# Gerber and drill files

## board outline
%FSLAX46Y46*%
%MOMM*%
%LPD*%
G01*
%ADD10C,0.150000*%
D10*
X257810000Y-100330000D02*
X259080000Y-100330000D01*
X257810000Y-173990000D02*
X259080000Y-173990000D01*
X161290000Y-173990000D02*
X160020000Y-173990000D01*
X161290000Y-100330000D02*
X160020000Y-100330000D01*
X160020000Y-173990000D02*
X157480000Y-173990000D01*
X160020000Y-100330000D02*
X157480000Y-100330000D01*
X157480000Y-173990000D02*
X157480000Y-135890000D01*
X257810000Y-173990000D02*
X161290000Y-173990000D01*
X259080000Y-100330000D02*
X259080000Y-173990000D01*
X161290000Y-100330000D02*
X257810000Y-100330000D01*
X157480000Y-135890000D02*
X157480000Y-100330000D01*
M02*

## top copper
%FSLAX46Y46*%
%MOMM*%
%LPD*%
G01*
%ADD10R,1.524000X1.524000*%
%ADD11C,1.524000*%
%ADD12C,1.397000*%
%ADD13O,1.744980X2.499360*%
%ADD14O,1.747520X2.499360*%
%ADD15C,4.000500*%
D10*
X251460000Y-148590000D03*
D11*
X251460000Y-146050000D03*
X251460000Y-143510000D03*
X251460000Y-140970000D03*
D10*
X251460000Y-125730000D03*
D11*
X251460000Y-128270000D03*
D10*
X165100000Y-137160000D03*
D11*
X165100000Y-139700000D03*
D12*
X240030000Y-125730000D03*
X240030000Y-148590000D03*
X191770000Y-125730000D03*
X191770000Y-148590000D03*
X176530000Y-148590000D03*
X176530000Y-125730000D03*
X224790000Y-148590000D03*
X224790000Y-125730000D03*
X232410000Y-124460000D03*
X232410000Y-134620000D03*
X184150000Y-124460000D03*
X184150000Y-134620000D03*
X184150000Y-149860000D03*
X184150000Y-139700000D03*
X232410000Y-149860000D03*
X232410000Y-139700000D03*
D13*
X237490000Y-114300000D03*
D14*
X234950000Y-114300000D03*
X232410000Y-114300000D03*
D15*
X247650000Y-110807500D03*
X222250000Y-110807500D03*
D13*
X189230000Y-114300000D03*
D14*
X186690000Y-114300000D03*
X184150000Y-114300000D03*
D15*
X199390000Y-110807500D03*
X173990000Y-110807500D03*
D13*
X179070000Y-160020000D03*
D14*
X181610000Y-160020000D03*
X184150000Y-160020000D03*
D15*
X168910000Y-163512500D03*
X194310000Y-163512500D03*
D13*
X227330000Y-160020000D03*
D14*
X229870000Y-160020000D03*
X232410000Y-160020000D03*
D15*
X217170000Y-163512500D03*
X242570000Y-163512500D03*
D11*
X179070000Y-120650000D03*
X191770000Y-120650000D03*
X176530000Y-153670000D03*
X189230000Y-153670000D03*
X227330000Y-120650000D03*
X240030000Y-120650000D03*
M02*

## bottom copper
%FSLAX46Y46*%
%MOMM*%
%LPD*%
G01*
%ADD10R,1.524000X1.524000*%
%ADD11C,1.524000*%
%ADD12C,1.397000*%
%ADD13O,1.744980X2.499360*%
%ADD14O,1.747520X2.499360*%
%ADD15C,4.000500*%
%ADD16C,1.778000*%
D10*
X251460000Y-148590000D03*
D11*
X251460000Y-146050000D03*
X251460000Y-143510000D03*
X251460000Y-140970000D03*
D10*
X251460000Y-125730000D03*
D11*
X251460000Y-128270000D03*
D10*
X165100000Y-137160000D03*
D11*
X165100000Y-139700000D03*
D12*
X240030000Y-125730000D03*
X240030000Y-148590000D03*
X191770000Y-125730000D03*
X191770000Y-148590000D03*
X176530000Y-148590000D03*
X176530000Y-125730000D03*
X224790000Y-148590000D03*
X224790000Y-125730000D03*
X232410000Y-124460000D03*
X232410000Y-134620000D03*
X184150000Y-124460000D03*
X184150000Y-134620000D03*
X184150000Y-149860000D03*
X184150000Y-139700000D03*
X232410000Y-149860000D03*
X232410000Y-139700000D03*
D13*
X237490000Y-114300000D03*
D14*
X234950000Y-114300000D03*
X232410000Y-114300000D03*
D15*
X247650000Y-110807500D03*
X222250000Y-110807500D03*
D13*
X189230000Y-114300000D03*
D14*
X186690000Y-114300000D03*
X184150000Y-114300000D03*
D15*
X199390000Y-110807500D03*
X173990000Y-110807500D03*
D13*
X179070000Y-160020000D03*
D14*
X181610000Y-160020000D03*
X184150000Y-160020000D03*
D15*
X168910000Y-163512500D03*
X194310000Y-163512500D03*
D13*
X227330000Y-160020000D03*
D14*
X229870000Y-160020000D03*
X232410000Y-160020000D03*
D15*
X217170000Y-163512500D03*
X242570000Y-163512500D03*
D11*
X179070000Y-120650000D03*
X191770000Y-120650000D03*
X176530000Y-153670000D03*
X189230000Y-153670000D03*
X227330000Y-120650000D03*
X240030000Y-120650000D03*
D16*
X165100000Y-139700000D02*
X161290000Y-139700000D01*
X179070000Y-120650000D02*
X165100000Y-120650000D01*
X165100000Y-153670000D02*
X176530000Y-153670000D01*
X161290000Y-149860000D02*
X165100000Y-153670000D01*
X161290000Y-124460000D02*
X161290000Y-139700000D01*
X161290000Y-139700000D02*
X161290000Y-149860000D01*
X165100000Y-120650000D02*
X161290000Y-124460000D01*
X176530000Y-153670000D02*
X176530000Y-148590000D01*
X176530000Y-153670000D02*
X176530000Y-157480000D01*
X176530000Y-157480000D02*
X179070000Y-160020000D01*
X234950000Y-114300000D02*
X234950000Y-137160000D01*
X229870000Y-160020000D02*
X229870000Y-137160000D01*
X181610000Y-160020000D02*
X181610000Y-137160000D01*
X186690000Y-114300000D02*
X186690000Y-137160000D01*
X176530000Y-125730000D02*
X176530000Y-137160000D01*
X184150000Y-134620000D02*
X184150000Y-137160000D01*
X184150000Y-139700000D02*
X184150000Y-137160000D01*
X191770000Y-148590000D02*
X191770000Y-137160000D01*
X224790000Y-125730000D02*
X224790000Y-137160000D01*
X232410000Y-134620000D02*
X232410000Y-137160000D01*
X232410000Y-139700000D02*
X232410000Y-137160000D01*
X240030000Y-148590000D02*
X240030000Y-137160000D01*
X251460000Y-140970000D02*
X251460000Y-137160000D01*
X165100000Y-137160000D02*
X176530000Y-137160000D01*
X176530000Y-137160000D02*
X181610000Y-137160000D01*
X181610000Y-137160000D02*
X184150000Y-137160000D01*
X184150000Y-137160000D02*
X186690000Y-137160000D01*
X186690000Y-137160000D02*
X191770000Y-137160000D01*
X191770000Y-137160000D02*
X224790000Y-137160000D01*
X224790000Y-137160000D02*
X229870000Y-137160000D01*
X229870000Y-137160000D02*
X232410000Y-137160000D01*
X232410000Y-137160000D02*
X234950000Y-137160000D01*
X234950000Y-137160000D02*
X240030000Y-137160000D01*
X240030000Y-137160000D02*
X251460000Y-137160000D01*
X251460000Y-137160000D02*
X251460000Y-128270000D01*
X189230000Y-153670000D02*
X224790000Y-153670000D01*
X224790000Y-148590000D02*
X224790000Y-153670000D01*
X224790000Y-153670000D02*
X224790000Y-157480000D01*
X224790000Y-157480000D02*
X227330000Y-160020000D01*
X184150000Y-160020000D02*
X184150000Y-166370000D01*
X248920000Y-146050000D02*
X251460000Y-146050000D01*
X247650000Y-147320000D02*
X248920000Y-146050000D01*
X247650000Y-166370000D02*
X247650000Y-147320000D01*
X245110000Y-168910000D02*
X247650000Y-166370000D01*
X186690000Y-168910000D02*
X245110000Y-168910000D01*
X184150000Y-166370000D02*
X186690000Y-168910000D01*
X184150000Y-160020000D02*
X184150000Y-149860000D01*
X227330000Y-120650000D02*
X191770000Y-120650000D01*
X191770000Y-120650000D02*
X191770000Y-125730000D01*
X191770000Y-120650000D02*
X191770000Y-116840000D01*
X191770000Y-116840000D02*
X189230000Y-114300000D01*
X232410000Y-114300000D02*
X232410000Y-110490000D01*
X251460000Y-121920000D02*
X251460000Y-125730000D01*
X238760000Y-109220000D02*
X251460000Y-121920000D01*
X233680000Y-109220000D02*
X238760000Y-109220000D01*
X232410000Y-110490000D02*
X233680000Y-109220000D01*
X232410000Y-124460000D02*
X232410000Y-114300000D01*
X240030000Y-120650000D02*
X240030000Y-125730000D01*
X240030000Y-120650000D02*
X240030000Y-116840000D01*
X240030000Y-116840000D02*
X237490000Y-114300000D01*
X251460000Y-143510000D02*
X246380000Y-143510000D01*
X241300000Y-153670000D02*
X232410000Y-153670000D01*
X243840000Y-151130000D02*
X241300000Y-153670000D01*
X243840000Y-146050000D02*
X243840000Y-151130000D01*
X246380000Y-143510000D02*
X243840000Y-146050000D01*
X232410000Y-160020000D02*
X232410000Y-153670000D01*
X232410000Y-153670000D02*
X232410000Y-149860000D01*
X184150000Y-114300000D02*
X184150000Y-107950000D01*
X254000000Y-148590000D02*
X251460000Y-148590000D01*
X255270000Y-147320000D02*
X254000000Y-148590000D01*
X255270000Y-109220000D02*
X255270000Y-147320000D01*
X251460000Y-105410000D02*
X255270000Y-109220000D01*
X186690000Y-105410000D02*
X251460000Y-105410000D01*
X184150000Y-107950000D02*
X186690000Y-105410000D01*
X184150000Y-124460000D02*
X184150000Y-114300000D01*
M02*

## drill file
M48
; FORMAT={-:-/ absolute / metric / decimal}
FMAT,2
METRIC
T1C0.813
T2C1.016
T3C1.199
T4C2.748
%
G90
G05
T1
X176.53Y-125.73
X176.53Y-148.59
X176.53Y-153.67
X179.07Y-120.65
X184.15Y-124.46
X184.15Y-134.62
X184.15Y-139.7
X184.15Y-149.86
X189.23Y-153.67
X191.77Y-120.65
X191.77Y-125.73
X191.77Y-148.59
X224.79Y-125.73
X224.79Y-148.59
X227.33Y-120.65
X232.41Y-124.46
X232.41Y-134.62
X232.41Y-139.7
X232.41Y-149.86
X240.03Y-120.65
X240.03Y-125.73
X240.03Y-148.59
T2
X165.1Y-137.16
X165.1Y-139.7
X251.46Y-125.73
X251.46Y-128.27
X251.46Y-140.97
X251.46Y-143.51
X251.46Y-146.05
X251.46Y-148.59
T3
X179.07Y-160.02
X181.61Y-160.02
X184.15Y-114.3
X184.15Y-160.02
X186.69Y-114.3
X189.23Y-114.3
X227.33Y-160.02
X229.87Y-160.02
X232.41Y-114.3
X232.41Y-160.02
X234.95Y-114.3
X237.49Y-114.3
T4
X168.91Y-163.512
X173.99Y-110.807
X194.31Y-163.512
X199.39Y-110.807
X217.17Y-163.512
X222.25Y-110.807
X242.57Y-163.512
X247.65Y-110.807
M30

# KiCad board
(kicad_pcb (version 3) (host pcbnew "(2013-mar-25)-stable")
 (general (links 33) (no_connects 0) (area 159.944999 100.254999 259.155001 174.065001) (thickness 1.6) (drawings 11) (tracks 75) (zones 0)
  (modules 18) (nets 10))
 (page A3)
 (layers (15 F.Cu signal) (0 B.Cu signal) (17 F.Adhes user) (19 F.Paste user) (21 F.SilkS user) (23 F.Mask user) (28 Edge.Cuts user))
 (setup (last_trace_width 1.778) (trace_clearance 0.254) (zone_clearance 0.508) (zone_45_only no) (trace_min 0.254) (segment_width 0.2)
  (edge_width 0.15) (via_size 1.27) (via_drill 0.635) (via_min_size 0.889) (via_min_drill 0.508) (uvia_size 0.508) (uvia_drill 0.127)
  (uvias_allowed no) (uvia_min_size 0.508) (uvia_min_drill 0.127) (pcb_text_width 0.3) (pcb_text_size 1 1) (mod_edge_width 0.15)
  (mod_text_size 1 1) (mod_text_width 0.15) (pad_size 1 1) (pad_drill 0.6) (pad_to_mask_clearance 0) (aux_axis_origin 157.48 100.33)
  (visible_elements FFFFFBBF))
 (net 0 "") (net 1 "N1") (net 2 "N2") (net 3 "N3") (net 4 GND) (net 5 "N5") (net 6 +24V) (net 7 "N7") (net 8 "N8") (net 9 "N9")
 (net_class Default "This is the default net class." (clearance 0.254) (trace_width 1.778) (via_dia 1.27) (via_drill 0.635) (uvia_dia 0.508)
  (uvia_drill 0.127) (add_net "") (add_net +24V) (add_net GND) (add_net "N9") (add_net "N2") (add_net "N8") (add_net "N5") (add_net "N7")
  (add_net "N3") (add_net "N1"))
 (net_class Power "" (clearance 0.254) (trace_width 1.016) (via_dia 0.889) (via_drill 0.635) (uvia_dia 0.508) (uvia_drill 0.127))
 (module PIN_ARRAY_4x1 (layer F.Cu) (at 251.46 144.78 90)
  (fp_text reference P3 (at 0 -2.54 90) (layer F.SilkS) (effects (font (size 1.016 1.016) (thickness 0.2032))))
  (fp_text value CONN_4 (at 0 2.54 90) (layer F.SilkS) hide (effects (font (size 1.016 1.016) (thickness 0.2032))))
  (pad 1 thru_hole rect (at -3.81 0 90) (size 1.524 1.524) (drill 1.016) (layers *.Cu *.Mask F.SilkS) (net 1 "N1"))
  (pad 2 thru_hole circle (at -1.27 0 90) (size 1.524 1.524) (drill 1.016) (layers *.Cu *.Mask F.SilkS) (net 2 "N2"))
  (pad 3 thru_hole circle (at 1.27 0 90) (size 1.524 1.524) (drill 1.016) (layers *.Cu *.Mask F.SilkS) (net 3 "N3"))
  (pad 4 thru_hole circle (at 3.81 0 90) (size 1.524 1.524) (drill 1.016) (layers *.Cu *.Mask F.SilkS) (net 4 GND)))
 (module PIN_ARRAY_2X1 (layer F.Cu) (at 251.46 127 270)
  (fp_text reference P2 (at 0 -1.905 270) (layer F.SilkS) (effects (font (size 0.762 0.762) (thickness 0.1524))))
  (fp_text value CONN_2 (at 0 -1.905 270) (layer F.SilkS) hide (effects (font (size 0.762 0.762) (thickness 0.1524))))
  (pad 1 thru_hole rect (at -1.27 0 270) (size 1.524 1.524) (drill 1.016) (layers *.Cu *.Mask F.SilkS) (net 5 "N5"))
  (pad 2 thru_hole circle (at 1.27 0 270) (size 1.524 1.524) (drill 1.016) (layers *.Cu *.Mask F.SilkS) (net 4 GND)))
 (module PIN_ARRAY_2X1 (layer F.Cu) (at 165.1 138.43 270)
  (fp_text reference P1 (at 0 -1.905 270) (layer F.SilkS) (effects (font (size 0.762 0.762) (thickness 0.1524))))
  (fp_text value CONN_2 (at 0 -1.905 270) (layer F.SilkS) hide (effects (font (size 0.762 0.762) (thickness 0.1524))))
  (pad 1 thru_hole rect (at -1.27 0 270) (size 1.524 1.524) (drill 1.016) (layers *.Cu *.Mask F.SilkS) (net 4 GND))
  (pad 2 thru_hole circle (at 1.27 0 270) (size 1.524 1.524) (drill 1.016) (layers *.Cu *.Mask F.SilkS) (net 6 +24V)))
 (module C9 (layer F.Cu) (at 240.03 137.16 270)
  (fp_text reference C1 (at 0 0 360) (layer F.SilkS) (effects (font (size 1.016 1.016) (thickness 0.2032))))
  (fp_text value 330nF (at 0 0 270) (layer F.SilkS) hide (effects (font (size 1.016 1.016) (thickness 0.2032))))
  (pad 1 thru_hole circle (at -11.43 0 270) (size 1.397 1.397) (drill 0.8128) (layers *.Cu *.Mask F.SilkS) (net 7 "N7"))
  (pad 2 thru_hole circle (at 11.43 0 270) (size 1.397 1.397) (drill 0.8128) (layers *.Cu *.Mask F.SilkS) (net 4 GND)))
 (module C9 (layer F.Cu) (at 191.77 137.16 270)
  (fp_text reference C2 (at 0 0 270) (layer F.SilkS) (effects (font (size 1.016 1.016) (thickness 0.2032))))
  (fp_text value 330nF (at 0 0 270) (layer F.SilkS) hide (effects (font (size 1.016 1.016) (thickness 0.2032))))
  (pad 1 thru_hole circle (at -11.43 0 270) (size 1.397 1.397) (drill 0.8128) (layers *.Cu *.Mask F.SilkS) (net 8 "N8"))
  (pad 2 thru_hole circle (at 11.43 0 270) (size 1.397 1.397) (drill 0.8128) (layers *.Cu *.Mask F.SilkS) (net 4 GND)))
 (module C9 (layer F.Cu) (at 176.53 137.16 90)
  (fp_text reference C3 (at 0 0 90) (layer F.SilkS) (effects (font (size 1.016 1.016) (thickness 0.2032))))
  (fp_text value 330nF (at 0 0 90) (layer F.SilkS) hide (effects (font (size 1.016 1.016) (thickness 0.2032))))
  (pad 1 thru_hole circle (at -11.43 0 90) (size 1.397 1.397) (drill 0.8128) (layers *.Cu *.Mask F.SilkS) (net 6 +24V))
  (pad 2 thru_hole circle (at 11.43 0 90) (size 1.397 1.397) (drill 0.8128) (layers *.Cu *.Mask F.SilkS) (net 4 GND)))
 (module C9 (layer F.Cu) (at 224.79 137.16 90)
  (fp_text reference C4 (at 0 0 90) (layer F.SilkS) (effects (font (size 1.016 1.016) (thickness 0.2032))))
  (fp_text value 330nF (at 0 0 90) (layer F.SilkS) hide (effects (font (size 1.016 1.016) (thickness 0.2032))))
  (pad 1 thru_hole circle (at -11.43 0 90) (size 1.397 1.397) (drill 0.8128) (layers *.Cu *.Mask F.SilkS) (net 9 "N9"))
  (pad 2 thru_hole circle (at 11.43 0 90) (size 1.397 1.397) (drill 0.8128) (layers *.Cu *.Mask F.SilkS) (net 4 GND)))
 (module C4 (layer F.Cu) (at 232.41 129.54 270)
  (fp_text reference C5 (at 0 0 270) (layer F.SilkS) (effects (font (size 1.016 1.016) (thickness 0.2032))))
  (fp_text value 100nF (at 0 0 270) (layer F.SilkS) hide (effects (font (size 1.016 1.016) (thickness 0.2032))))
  (pad 1 thru_hole circle (at -5.08 0 270) (size 1.397 1.397) (drill 0.8128) (layers *.Cu *.Mask F.SilkS) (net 5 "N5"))
  (pad 2 thru_hole circle (at 5.08 0 270) (size 1.397 1.397) (drill 0.8128) (layers *.Cu *.Mask F.SilkS) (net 4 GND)))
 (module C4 (layer F.Cu) (at 184.15 129.54 270)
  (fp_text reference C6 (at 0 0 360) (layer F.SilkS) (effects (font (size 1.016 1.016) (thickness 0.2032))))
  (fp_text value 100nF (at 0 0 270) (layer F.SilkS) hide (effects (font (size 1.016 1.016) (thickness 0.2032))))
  (pad 1 thru_hole circle (at -5.08 0 270) (size 1.397 1.397) (drill 0.8128) (layers *.Cu *.Mask F.SilkS) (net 1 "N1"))
  (pad 2 thru_hole circle (at 5.08 0 270) (size 1.397 1.397) (drill 0.8128) (layers *.Cu *.Mask F.SilkS) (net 4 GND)))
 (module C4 (layer F.Cu) (at 184.15 144.78 90)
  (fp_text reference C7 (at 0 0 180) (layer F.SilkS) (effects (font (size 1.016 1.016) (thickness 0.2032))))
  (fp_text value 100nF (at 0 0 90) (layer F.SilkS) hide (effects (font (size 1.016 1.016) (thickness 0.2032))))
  (pad 1 thru_hole circle (at -5.08 0 90) (size 1.397 1.397) (drill 0.8128) (layers *.Cu *.Mask F.SilkS) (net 2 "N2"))
  (pad 2 thru_hole circle (at 5.08 0 90) (size 1.397 1.397) (drill 0.8128) (layers *.Cu *.Mask F.SilkS) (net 4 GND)))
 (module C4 (layer F.Cu) (at 232.41 144.78 90)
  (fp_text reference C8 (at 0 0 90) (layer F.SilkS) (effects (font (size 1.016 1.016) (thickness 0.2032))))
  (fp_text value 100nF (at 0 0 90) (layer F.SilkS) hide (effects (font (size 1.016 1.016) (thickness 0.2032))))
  (pad 1 thru_hole circle (at -5.08 0 90) (size 1.397 1.397) (drill 0.8128) (layers *.Cu *.Mask F.SilkS) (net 3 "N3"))
  (pad 2 thru_hole circle (at 5.08 0 90) (size 1.397 1.397) (drill 0.8128) (layers *.Cu *.Mask F.SilkS) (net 4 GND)))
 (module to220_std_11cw (layer F.Cu) (at 234.95 114.3)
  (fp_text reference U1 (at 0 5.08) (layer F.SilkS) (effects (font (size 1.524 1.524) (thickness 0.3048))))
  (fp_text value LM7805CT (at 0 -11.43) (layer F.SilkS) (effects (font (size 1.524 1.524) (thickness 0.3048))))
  (pad 1 thru_hole oval (at 2.54 0) (size 1.74498 2.49936) (drill 1.19888) (layers *.Cu *.Mask F.SilkS) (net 7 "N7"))
  (pad 2 thru_hole oval (at 0 0) (size 1.74752 2.49936) (drill 1.19888) (layers *.Cu *.Mask F.SilkS) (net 4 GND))
  (pad 3 thru_hole oval (at -2.54 0) (size 1.74752 2.49936) (drill 1.19888) (layers *.Cu *.Mask F.SilkS) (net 5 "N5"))
  (pad "" thru_hole circle (at 12.7 -3.4925) (size 4.0005 4.0005) (drill 2.74828) (layers *.Cu *.Mask F.SilkS))
  (pad "" thru_hole circle (at -12.7 -3.4925) (size 4.0005 4.0005) (drill 2.74828) (layers *.Cu *.Mask F.SilkS)))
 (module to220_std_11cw (layer F.Cu) (at 186.69 114.3)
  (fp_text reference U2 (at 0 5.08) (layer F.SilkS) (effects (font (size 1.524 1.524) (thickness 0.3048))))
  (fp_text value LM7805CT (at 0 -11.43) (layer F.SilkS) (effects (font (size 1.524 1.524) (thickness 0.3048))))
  (pad 1 thru_hole oval (at 2.54 0) (size 1.74498 2.49936) (drill 1.19888) (layers *.Cu *.Mask F.SilkS) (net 8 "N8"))
  (pad 2 thru_hole oval (at 0 0) (size 1.74752 2.49936) (drill 1.19888) (layers *.Cu *.Mask F.SilkS) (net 4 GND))
  (pad 3 thru_hole oval (at -2.54 0) (size 1.74752 2.49936) (drill 1.19888) (layers *.Cu *.Mask F.SilkS) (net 1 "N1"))
  (pad "" thru_hole circle (at 12.7 -3.4925) (size 4.0005 4.0005) (drill 2.74828) (layers *.Cu *.Mask F.SilkS))
  (pad "" thru_hole circle (at -12.7 -3.4925) (size 4.0005 4.0005) (drill 2.74828) (layers *.Cu *.Mask F.SilkS)))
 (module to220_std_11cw (layer F.Cu) (at 181.61 160.02 180)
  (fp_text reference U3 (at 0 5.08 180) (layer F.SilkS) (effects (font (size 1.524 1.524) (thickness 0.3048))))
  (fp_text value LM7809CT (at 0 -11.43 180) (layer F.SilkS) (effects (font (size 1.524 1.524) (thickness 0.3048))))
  (pad 1 thru_hole oval (at 2.54 0 180) (size 1.74498 2.49936) (drill 1.19888) (layers *.Cu *.Mask F.SilkS) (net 6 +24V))
  (pad 2 thru_hole oval (at 0 0 180) (size 1.74752 2.49936) (drill 1.19888) (layers *.Cu *.Mask F.SilkS) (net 4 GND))
  (pad 3 thru_hole oval (at -2.54 0 180) (size 1.74752 2.49936) (drill 1.19888) (layers *.Cu *.Mask F.SilkS) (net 2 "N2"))
  (pad "" thru_hole circle (at 12.7 -3.4925 180) (size 4.0005 4.0005) (drill 2.74828) (layers *.Cu *.Mask F.SilkS))
  (pad "" thru_hole circle (at -12.7 -3.4925 180) (size 4.0005 4.0005) (drill 2.74828) (layers *.Cu *.Mask F.SilkS)))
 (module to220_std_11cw (layer F.Cu) (at 229.87 160.02 180)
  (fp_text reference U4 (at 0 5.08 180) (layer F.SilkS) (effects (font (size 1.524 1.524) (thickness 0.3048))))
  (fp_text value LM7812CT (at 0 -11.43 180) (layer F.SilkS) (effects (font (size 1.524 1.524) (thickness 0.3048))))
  (pad 1 thru_hole oval (at 2.54 0 180) (size 1.74498 2.49936) (drill 1.19888) (layers *.Cu *.Mask F.SilkS) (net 9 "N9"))
  (pad 2 thru_hole oval (at 0 0 180) (size 1.74752 2.49936) (drill 1.19888) (layers *.Cu *.Mask F.SilkS) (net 4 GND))
  (pad 3 thru_hole oval (at -2.54 0 180) (size 1.74752 2.49936) (drill 1.19888) (layers *.Cu *.Mask F.SilkS) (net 3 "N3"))
  (pad "" thru_hole circle (at 12.7 -3.4925 180) (size 4.0005 4.0005) (drill 2.74828) (layers *.Cu *.Mask F.SilkS))
  (pad "" thru_hole circle (at -12.7 -3.4925 180) (size 4.0005 4.0005) (drill 2.74828) (layers *.Cu *.Mask F.SilkS)))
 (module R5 (layer F.Cu) (at 185.42 120.65) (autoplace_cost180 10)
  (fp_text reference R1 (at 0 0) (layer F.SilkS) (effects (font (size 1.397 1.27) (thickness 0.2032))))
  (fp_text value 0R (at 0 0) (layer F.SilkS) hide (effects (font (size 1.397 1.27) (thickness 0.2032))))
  (pad 1 thru_hole circle (at -6.35 0) (size 1.524 1.524) (drill 0.8128) (layers *.Cu *.Mask F.SilkS) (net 6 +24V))
  (pad 2 thru_hole circle (at 6.35 0) (size 1.524 1.524) (drill 0.8128) (layers *.Cu *.Mask F.SilkS) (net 8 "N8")))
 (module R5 (layer F.Cu) (at 182.88 153.67) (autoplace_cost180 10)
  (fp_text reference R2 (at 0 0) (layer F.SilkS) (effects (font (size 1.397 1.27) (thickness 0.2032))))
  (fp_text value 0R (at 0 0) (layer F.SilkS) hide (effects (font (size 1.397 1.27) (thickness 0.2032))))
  (pad 1 thru_hole circle (at -6.35 0) (size 1.524 1.524) (drill 0.8128) (layers *.Cu *.Mask F.SilkS) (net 6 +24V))
  (pad 2 thru_hole circle (at 6.35 0) (size 1.524 1.524) (drill 0.8128) (layers *.Cu *.Mask F.SilkS) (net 9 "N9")))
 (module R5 (layer F.Cu) (at 233.68 120.65) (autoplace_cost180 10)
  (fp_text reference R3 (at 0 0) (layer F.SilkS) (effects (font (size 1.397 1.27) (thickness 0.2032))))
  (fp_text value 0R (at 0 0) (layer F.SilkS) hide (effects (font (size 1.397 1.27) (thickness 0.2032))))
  (pad 1 thru_hole circle (at -6.35 0) (size 1.524 1.524) (drill 0.8128) (layers *.Cu *.Mask F.SilkS) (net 8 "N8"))
  (pad 2 thru_hole circle (at 6.35 0) (size 1.524 1.524) (drill 0.8128) (layers *.Cu *.Mask F.SilkS) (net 7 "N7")))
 (gr_line (start 257.81 100.33) (end 259.08 100.33) (angle 90) (layer Edge.Cuts) (width 0.15))
 (gr_line (start 257.81 173.99) (end 259.08 173.99) (angle 90) (layer Edge.Cuts) (width 0.15))
 (gr_line (start 161.29 173.99) (end 160.02 173.99) (angle 90) (layer Edge.Cuts) (width 0.15))
 (gr_line (start 161.29 100.33) (end 160.02 100.33) (angle 90) (layer Edge.Cuts) (width 0.15))
 (gr_line (start 160.02 173.99) (end 157.48 173.99) (angle 90) (layer Edge.Cuts) (width 0.15))
 (gr_line (start 160.02 100.33) (end 157.48 100.33) (angle 90) (layer Edge.Cuts) (width 0.15))
 (gr_line (start 157.48 173.99) (end 157.48 135.89) (angle 90) (layer Edge.Cuts) (width 0.15))
 (gr_line (start 257.81 173.99) (end 161.29 173.99) (angle 90) (layer Edge.Cuts) (width 0.15))
 (gr_line (start 259.08 100.33) (end 259.08 173.99) (angle 90) (layer Edge.Cuts) (width 0.15))
 (gr_line (start 161.29 100.33) (end 257.81 100.33) (angle 90) (layer Edge.Cuts) (width 0.15))
 (gr_line (start 157.48 135.89) (end 157.48 100.33) (angle 90) (layer Edge.Cuts) (width 0.15))
 (segment (start 165.1 139.7) (end 161.29 139.7) (width 1.778) (layer B.Cu) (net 6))
 (segment (start 179.07 120.65) (end 165.1 120.65) (width 1.778) (layer B.Cu) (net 6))
 (segment (start 165.1 153.67) (end 176.53 153.67) (width 1.778) (layer B.Cu) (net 6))
 (segment (start 161.29 149.86) (end 165.1 153.67) (width 1.778) (layer B.Cu) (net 6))
 (segment (start 161.29 124.46) (end 161.29 139.7) (width 1.778) (layer B.Cu) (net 6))
 (segment (start 161.29 139.7) (end 161.29 149.86) (width 1.778) (layer B.Cu) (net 6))
 (segment (start 165.1 120.65) (end 161.29 124.46) (width 1.778) (layer B.Cu) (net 6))
 (segment (start 176.53 153.67) (end 176.53 148.59) (width 1.778) (layer B.Cu) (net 6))
 (segment (start 176.53 153.67) (end 176.53 157.48) (width 1.778) (layer B.Cu) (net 6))
 (segment (start 176.53 157.48) (end 179.07 160.02) (width 1.778) (layer B.Cu) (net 6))
 (segment (start 234.95 114.3) (end 234.95 137.16) (width 1.778) (layer B.Cu) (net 4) (status 400000))
 (segment (start 229.87 160.02) (end 229.87 137.16) (width 1.778) (layer B.Cu) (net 4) (status 400000))
 (segment (start 181.61 160.02) (end 181.61 137.16) (width 1.778) (layer B.Cu) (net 4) (status 400000))
 (segment (start 186.69 114.3) (end 186.69 137.16) (width 1.778) (layer B.Cu) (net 4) (status 400000))
 (segment (start 176.53 125.73) (end 176.53 137.16) (width 1.778) (layer B.Cu) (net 4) (status 400000))
 (segment (start 184.15 134.62) (end 184.15 137.16) (width 1.778) (layer B.Cu) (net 4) (status 400000))
 (segment (start 184.15 139.7) (end 184.15 137.16) (width 1.778) (layer B.Cu) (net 4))
 (segment (start 191.77 148.59) (end 191.77 137.16) (width 1.778) (layer B.Cu) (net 4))
 (segment (start 224.79 125.73) (end 224.79 137.16) (width 1.778) (layer B.Cu) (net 4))
 (segment (start 232.41 134.62) (end 232.41 137.16) (width 1.778) (layer B.Cu) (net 4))
 (segment (start 232.41 139.7) (end 232.41 137.16) (width 1.778) (layer B.Cu) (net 4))
 (segment (start 240.03 148.59) (end 240.03 137.16) (width 1.778) (layer B.Cu) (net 4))
 (segment (start 251.46 140.97) (end 251.46 137.16) (width 1.778) (layer B.Cu) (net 4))
 (segment (start 165.1 137.16) (end 176.53 137.16) (width 1.778) (layer B.Cu) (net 4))
 (segment (start 176.53 137.16) (end 181.61 137.16) (width 1.778) (layer B.Cu) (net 4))
 (segment (start 181.61 137.16) (end 184.15 137.16) (width 1.778) (layer B.Cu) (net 4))
 (segment (start 184.15 137.16) (end 186.69 137.16) (width 1.778) (layer B.Cu) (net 4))
 (segment (start 186.69 137.16) (end 191.77 137.16) (width 1.778) (layer B.Cu) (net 4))
 (segment (start 191.77 137.16) (end 224.79 137.16) (width 1.778) (layer B.Cu) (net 4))
 (segment (start 224.79 137.16) (end 229.87 137.16) (width 1.778) (layer B.Cu) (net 4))
 (segment (start 229.87 137.16) (end 232.41 137.16) (width 1.778) (layer B.Cu) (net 4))
 (segment (start 232.41 137.16) (end 234.95 137.16) (width 1.778) (layer B.Cu) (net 4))
 (segment (start 234.95 137.16) (end 240.03 137.16) (width 1.778) (layer B.Cu) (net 4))
 (segment (start 240.03 137.16) (end 251.46 137.16) (width 1.778) (layer B.Cu) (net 4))
 (segment (start 251.46 137.16) (end 251.46 128.27) (width 1.778) (layer B.Cu) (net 4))
 (segment (start 189.23 153.67) (end 224.79 153.67) (width 1.778) (layer B.Cu) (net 9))
 (segment (start 224.79 148.59) (end 224.79 153.67) (width 1.778) (layer B.Cu) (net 9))
 (segment (start 224.79 153.67) (end 224.79 157.48) (width 1.778) (layer B.Cu) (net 9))
 (segment (start 224.79 157.48) (end 227.33 160.02) (width 1.778) (layer B.Cu) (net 9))
 (segment (start 184.15 160.02) (end 184.15 166.37) (width 1.778) (layer B.Cu) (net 2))
 (segment (start 248.92 146.05) (end 251.46 146.05) (width 1.778) (layer B.Cu) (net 2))
 (segment (start 247.65 147.32) (end 248.92 146.05) (width 1.778) (layer B.Cu) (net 2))
 (segment (start 247.65 166.37) (end 247.65 147.32) (width 1.778) (layer B.Cu) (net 2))
 (segment (start 245.11 168.91) (end 247.65 166.37) (width 1.778) (layer B.Cu) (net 2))
 (segment (start 186.69 168.91) (end 245.11 168.91) (width 1.778) (layer B.Cu) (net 2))
 (segment (start 184.15 166.37) (end 186.69 168.91) (width 1.778) (layer B.Cu) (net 2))
 (segment (start 184.15 160.02) (end 184.15 149.86) (width 1.778) (layer B.Cu) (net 2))
 (segment (start 227.33 120.65) (end 191.77 120.65) (width 1.778) (layer B.Cu) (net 8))
 (segment (start 191.77 120.65) (end 191.77 125.73) (width 1.778) (layer B.Cu) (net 8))
 (segment (start 191.77 120.65) (end 191.77 116.84) (width 1.778) (layer B.Cu) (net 8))
 (segment (start 191.77 116.84) (end 189.23 114.3) (width 1.778) (layer B.Cu) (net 8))
 (segment (start 232.41 114.3) (end 232.41 110.49) (width 1.778) (layer B.Cu) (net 5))
 (segment (start 251.46 121.92) (end 251.46 125.73) (width 1.778) (layer B.Cu) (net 5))
 (segment (start 238.76 109.22) (end 251.46 121.92) (width 1.778) (layer B.Cu) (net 5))
 (segment (start 233.68 109.22) (end 238.76 109.22) (width 1.778) (layer B.Cu) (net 5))
 (segment (start 232.41 110.49) (end 233.68 109.22) (width 1.778) (layer B.Cu) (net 5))
 (segment (start 232.41 124.46) (end 232.41 114.3) (width 1.778) (layer B.Cu) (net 5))
 (segment (start 240.03 120.65) (end 240.03 125.73) (width 1.778) (layer B.Cu) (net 7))
 (segment (start 240.03 120.65) (end 240.03 116.84) (width 1.778) (layer B.Cu) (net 7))
 (segment (start 240.03 116.84) (end 237.49 114.3) (width 1.778) (layer B.Cu) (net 7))
 (segment (start 251.46 143.51) (end 246.38 143.51) (width 1.778) (layer B.Cu) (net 3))
 (segment (start 241.3 153.67) (end 232.41 153.67) (width 1.778) (layer B.Cu) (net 3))
 (segment (start 243.84 151.13) (end 241.3 153.67) (width 1.778) (layer B.Cu) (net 3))
 (segment (start 243.84 146.05) (end 243.84 151.13) (width 1.778) (layer B.Cu) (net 3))
 (segment (start 246.38 143.51) (end 243.84 146.05) (width 1.778) (layer B.Cu) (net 3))
 (segment (start 232.41 160.02) (end 232.41 153.67) (width 1.778) (layer B.Cu) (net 3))
 (segment (start 232.41 153.67) (end 232.41 149.86) (width 1.778) (layer B.Cu) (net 3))
 (segment (start 184.15 114.3) (end 184.15 107.95) (width 1.778) (layer B.Cu) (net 1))
 (segment (start 254 148.59) (end 251.46 148.59) (width 1.778) (layer B.Cu) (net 1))
 (segment (start 255.27 147.32) (end 254 148.59) (width 1.778) (layer B.Cu) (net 1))
 (segment (start 255.27 109.22) (end 255.27 147.32) (width 1.778) (layer B.Cu) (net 1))
 (segment (start 251.46 105.41) (end 255.27 109.22) (width 1.778) (layer B.Cu) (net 1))
 (segment (start 186.69 105.41) (end 251.46 105.41) (width 1.778) (layer B.Cu) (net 1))
 (segment (start 184.15 107.95) (end 186.69 105.41) (width 1.778) (layer B.Cu) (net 1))
 (segment (start 184.15 124.46) (end 184.15 114.3) (width 1.778) (layer B.Cu) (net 1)))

